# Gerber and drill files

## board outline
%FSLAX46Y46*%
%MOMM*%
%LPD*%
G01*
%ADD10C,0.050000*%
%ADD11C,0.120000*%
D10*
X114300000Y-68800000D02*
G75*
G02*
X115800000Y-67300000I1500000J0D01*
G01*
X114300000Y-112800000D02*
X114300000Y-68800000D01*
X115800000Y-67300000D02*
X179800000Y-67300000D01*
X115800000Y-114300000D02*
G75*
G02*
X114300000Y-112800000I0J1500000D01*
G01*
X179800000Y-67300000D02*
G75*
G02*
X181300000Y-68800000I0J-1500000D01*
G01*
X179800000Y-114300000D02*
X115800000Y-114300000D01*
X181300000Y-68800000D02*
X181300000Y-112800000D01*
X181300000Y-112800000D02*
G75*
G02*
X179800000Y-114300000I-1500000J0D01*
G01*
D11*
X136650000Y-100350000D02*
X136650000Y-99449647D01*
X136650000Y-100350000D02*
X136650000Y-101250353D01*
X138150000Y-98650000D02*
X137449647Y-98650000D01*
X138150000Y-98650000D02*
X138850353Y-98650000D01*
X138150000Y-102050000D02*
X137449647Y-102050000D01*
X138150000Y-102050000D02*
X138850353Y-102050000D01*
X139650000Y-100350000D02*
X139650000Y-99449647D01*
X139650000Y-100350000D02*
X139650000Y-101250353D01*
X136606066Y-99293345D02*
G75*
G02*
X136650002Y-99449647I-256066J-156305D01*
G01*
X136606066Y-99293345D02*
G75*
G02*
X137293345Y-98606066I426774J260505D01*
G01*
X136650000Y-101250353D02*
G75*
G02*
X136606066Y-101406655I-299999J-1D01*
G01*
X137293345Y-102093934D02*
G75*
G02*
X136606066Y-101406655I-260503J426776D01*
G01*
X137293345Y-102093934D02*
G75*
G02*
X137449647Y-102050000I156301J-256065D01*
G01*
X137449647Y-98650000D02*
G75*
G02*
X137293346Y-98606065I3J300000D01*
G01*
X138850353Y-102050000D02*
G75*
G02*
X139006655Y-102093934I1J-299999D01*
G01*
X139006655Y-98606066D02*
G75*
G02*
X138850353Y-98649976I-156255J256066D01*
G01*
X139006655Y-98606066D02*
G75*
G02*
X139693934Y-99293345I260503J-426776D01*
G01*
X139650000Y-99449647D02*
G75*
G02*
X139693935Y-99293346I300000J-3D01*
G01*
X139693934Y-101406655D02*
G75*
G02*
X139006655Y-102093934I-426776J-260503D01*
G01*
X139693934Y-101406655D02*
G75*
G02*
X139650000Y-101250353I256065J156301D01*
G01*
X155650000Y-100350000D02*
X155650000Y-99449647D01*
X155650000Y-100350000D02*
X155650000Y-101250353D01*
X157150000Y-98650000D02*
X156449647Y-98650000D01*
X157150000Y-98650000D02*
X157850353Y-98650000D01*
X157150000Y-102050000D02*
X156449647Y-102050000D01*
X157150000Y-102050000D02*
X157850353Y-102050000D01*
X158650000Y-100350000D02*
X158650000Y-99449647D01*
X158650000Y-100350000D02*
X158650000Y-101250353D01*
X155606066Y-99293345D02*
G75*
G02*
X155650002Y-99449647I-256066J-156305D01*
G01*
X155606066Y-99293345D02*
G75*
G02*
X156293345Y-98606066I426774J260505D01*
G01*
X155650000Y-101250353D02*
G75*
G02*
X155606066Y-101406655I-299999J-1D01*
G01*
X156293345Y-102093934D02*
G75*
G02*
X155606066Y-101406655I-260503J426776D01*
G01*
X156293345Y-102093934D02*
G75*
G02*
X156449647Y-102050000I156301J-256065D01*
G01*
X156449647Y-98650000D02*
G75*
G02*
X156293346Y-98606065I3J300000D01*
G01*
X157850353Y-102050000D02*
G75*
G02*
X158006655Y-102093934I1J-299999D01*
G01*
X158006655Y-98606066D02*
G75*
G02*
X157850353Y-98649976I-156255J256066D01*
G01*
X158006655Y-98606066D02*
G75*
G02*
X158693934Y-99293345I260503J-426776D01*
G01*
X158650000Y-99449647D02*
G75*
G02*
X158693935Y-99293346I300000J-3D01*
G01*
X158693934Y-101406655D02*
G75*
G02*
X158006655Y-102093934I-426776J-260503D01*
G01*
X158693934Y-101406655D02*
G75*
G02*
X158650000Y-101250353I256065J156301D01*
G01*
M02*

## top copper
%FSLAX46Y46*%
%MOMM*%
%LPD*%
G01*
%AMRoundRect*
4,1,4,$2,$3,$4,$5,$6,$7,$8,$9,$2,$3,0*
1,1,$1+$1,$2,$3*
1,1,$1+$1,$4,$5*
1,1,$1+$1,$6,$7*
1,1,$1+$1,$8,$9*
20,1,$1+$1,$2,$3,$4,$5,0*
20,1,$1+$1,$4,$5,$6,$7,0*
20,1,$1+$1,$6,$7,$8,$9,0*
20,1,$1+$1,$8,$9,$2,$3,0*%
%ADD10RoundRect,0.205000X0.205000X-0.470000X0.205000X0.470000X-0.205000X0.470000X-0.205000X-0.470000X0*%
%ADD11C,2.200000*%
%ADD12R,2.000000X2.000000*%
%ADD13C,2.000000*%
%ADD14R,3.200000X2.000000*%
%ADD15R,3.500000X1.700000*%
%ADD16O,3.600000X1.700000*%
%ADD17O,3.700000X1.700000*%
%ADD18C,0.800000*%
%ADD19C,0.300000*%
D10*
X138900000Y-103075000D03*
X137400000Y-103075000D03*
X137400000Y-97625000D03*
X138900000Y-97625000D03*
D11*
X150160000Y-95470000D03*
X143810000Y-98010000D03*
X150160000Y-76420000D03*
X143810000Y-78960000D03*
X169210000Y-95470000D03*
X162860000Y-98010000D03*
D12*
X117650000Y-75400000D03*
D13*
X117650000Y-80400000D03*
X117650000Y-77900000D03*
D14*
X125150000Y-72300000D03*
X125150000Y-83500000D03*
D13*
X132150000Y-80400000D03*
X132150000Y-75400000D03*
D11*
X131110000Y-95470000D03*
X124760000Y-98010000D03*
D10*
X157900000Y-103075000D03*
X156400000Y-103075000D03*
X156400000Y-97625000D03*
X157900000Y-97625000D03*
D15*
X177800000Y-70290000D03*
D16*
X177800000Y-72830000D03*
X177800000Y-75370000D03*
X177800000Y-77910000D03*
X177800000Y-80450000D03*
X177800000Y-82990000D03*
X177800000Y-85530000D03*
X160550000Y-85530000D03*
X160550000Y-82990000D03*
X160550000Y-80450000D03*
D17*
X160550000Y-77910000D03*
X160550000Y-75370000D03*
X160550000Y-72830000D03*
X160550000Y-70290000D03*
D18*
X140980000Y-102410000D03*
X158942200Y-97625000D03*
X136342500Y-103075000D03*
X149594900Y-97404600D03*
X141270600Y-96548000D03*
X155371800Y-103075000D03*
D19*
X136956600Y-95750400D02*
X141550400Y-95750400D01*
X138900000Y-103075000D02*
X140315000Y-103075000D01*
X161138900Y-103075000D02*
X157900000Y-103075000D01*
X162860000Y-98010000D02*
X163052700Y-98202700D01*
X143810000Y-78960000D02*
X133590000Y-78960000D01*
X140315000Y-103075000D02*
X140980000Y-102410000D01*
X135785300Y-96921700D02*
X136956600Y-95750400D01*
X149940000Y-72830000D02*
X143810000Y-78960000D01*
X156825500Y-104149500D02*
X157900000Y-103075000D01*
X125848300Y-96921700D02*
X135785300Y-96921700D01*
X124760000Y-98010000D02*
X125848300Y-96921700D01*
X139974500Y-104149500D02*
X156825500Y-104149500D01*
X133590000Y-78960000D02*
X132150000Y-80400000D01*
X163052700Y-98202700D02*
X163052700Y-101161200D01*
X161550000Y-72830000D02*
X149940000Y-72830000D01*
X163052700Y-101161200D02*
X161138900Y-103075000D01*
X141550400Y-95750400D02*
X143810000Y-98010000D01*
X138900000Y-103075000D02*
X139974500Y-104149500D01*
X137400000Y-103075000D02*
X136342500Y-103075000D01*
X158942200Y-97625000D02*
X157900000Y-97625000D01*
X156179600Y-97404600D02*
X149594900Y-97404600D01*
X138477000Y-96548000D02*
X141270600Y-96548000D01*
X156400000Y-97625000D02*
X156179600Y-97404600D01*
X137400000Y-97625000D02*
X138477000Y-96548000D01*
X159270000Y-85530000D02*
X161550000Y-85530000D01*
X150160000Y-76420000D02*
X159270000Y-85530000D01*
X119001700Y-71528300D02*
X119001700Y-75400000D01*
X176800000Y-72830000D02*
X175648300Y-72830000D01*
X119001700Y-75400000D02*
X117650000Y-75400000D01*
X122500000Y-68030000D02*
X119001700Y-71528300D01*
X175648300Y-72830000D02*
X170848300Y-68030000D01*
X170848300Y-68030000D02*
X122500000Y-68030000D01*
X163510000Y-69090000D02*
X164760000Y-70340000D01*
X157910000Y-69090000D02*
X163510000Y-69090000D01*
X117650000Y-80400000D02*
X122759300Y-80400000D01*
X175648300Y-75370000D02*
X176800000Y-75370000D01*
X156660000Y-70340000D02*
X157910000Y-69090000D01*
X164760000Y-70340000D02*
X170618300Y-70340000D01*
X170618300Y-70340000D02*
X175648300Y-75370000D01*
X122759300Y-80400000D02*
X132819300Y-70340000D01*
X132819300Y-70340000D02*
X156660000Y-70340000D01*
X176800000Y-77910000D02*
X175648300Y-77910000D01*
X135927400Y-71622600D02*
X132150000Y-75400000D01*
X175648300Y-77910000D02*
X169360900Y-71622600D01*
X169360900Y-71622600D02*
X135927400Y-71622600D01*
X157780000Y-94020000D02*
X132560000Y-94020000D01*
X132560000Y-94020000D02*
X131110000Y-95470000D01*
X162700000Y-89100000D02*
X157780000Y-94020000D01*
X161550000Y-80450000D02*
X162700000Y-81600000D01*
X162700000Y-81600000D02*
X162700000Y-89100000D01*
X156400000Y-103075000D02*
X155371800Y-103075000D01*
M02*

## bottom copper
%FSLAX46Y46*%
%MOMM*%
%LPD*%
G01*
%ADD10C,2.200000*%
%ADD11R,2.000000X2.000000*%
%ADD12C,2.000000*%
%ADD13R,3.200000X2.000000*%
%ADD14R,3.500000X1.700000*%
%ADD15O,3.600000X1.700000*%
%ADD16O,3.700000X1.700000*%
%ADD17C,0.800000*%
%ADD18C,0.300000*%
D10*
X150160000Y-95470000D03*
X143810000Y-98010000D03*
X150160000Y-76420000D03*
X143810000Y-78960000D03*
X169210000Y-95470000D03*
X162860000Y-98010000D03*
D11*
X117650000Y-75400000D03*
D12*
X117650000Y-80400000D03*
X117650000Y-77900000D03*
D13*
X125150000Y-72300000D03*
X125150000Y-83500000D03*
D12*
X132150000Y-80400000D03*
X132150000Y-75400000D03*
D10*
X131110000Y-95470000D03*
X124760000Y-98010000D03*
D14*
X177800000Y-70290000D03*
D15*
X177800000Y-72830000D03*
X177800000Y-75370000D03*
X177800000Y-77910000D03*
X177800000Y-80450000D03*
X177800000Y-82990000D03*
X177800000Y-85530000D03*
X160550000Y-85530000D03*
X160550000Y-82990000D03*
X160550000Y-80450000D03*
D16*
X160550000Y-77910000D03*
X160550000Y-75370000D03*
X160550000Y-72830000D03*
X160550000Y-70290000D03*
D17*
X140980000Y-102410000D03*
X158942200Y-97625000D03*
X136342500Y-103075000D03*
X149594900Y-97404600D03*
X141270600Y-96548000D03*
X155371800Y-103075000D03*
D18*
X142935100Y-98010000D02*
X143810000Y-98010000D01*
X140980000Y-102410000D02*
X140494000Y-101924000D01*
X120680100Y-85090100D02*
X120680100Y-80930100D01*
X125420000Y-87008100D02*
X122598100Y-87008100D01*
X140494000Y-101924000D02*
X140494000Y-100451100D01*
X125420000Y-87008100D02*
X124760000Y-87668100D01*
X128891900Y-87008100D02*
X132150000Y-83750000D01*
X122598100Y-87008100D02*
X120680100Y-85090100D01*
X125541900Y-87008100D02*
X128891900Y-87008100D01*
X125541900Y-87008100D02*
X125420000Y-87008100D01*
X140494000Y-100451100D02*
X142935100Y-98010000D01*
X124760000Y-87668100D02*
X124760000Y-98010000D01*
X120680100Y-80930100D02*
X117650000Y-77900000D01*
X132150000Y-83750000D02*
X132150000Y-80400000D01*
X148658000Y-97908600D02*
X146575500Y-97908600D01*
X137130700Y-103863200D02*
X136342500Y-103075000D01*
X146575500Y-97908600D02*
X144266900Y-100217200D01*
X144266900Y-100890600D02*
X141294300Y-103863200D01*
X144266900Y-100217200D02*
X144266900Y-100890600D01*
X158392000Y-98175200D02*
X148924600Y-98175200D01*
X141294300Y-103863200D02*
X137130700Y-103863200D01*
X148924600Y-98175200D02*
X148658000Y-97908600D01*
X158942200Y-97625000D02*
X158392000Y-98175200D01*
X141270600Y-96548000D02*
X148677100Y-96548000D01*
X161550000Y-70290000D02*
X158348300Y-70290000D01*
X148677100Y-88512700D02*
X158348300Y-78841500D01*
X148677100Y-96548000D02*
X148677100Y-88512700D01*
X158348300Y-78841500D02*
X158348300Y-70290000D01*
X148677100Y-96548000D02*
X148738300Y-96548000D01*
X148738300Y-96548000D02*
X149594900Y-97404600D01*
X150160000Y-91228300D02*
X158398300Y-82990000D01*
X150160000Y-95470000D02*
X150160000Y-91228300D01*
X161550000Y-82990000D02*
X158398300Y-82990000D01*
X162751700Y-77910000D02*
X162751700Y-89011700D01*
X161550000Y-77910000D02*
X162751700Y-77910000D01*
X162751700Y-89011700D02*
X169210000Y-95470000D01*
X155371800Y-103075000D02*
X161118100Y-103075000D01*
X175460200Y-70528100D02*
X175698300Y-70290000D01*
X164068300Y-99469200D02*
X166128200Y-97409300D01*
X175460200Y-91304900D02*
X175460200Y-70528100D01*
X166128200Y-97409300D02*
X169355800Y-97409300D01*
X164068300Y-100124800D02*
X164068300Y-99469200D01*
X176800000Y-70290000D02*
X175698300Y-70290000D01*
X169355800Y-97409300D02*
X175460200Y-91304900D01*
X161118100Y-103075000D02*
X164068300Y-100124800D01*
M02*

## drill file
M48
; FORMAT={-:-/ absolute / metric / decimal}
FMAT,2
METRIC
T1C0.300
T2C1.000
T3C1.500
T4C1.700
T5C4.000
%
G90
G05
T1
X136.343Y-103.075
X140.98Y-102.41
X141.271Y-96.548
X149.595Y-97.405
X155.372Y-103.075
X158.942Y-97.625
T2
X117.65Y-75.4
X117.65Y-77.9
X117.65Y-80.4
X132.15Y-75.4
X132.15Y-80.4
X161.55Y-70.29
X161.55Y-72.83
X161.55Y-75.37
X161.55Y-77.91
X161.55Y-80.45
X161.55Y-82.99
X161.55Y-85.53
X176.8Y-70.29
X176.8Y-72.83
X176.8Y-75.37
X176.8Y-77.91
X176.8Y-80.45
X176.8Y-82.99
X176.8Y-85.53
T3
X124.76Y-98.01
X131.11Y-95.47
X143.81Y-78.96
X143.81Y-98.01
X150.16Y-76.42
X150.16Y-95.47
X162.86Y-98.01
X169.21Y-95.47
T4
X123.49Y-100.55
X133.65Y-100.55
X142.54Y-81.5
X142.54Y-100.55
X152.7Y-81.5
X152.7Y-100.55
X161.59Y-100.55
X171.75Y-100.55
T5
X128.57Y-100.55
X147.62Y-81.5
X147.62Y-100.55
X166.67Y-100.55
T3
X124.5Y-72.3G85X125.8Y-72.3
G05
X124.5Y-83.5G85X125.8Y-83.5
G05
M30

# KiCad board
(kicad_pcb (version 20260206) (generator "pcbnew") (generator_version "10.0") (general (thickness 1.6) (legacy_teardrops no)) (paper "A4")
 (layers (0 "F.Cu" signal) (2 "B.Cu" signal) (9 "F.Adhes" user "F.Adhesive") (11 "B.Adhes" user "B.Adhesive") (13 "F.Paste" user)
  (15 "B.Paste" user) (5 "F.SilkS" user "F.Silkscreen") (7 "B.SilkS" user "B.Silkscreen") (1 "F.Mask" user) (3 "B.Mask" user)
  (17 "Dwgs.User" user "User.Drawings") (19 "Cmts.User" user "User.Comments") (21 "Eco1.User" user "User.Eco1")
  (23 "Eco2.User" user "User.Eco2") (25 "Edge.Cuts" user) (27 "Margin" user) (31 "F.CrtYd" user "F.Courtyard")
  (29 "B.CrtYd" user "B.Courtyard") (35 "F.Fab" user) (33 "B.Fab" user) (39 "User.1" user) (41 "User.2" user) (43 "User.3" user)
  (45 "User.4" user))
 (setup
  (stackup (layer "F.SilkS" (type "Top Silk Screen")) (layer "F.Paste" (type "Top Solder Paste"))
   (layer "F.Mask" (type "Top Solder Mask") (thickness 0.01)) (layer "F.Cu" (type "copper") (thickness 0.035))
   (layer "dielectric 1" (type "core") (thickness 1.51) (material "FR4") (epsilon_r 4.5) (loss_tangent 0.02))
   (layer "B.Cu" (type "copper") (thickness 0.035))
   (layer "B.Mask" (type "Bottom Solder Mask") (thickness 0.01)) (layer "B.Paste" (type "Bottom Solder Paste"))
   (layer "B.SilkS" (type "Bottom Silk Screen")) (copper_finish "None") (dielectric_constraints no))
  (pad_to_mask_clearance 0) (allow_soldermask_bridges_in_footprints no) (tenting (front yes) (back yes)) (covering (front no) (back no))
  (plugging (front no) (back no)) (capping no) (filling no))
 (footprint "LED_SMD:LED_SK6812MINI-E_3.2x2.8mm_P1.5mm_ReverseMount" (layer "F.Cu") (at 138.15 100.35 90)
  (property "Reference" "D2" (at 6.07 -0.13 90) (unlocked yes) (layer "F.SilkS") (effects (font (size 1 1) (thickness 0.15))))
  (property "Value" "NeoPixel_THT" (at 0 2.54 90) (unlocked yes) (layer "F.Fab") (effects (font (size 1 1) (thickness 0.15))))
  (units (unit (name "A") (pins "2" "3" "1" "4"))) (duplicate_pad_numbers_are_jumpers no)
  (fp_line (start 0 -1.5) (end 0.900353 -1.5) (stroke (width 0.12) (type solid)) (layer "Edge.Cuts"))
  (fp_line (start 0 -1.5) (end -0.900353 -1.5) (stroke (width 0.12) (type solid)) (layer "Edge.Cuts"))
  (fp_line (start 1.7 0) (end 1.7 -0.700353) (stroke (width 0.12) (type solid)) (layer "Edge.Cuts"))
  (fp_line (start 1.7 0) (end 1.7 0.700353) (stroke (width 0.12) (type solid)) (layer "Edge.Cuts"))
  (fp_line (start -1.7 0) (end -1.7 -0.700353) (stroke (width 0.12) (type solid)) (layer "Edge.Cuts"))
  (fp_line (start -1.7 0) (end -1.7 0.700353) (stroke (width 0.12) (type solid)) (layer "Edge.Cuts"))
  (fp_line (start 0 1.5) (end 0.900353 1.5) (stroke (width 0.12) (type solid)) (layer "Edge.Cuts"))
  (fp_line (start 0 1.5) (end -0.900353 1.5) (stroke (width 0.12) (type solid)) (layer "Edge.Cuts"))
  (fp_arc (start 1.056655 -1.543934) (mid 0.981532 -1.511192) (end 0.900353 -1.5) (stroke (width 0.12) (type solid)) (layer "Edge.Cuts"))
  (fp_arc (start 1.056655 -1.543934) (mid 1.670711 -1.470711) (end 1.743934 -0.856655) (stroke (width 0.12) (type solid))
   (layer "Edge.Cuts"))
  (fp_arc (start -0.900353 -1.5) (mid -0.981532 -1.511192) (end -1.056655 -1.543934) (stroke (width 0.12) (type solid)) (layer "Edge.Cuts"))
  (fp_arc (start -1.743934 -0.856655) (mid -1.670711 -1.470711) (end -1.056655 -1.543934) (stroke (width 0.12) (type solid))
   (layer "Edge.Cuts"))
  (fp_arc (start -1.743934 -0.856655) (mid -1.711192 -0.781532) (end -1.7 -0.700353) (stroke (width 0.12) (type solid)) (layer "Edge.Cuts"))
  (fp_arc (start 1.7 -0.700353) (mid 1.711192 -0.781532) (end 1.743934 -0.856655) (stroke (width 0.12) (type solid)) (layer "Edge.Cuts"))
  (fp_arc (start -1.7 0.700353) (mid -1.711192 0.781532) (end -1.743934 0.856655) (stroke (width 0.12) (type solid)) (layer "Edge.Cuts"))
  (fp_arc (start 1.743934 0.856655) (mid 1.711192 0.781532) (end 1.7 0.700353) (stroke (width 0.12) (type solid)) (layer "Edge.Cuts"))
  (fp_arc (start 1.743934 0.856655) (mid 1.670711 1.470711) (end 1.056655 1.543934) (stroke (width 0.12) (type solid)) (layer "Edge.Cuts"))
  (fp_arc (start 0.900353 1.5) (mid 0.981532 1.511192) (end 1.056655 1.543934) (stroke (width 0.12) (type solid)) (layer "Edge.Cuts"))
  (fp_arc (start -1.056655 1.543934) (mid -1.670711 1.470711) (end -1.743934 0.856655) (stroke (width 0.12) (type solid))
   (layer "Edge.Cuts"))
  (fp_arc (start -1.056655 1.543934) (mid -0.981532 1.511192) (end -0.900353 1.5) (stroke (width 0.12) (type solid)) (layer "Edge.Cuts"))
  (pad "1" smd roundrect (at -2.725 0.75 90) (size 1.35 0.82) (layers "F.Cu" "F.Mask" "F.Paste") (roundrect_rratio 0.25) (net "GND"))
  (pad "2" smd roundrect (at -2.725 -0.75 90) (size 1.35 0.82) (layers "F.Cu" "F.Mask" "F.Paste") (roundrect_rratio 0.25)
   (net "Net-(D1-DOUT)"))
  (pad "3" smd roundrect (at 2.725 -0.75 90) (size 1.35 0.82) (layers "F.Cu" "F.Mask" "F.Paste") (roundrect_rratio 0.25) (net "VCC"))
  (pad "4" smd roundrect (at 2.725 0.75 90) (size 1.35 0.82) (layers "F.Cu" "F.Mask" "F.Paste") (roundrect_rratio 0.25)
   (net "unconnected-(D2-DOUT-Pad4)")))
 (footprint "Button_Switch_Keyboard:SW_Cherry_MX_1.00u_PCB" (layer "F.Cu") (at 150.16 95.47)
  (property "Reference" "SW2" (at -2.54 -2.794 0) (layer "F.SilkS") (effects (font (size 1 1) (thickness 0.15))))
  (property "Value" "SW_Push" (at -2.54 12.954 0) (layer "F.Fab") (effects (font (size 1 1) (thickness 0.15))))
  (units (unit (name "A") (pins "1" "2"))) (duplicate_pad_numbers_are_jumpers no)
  (pad "" np_thru_hole circle (at -7.62 5.08) (size 1.7 1.7) (drill 1.7) (layers "*.Cu" "*.Mask"))
  (pad "" np_thru_hole circle (at -2.54 5.08) (size 4 4) (drill 4) (layers "*.Cu" "*.Mask"))
  (pad "" np_thru_hole circle (at 2.54 5.08) (size 1.7 1.7) (drill 1.7) (layers "*.Cu" "*.Mask"))
  (pad "1" thru_hole circle (at 0 0) (size 2.2 2.2) (drill 1.5) (layers "*.Cu" "*.Mask") (remove_unused_layers no)
   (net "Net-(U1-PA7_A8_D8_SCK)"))
  (pad "2" thru_hole circle (at -6.35 2.54) (size 2.2 2.2) (drill 1.5) (layers "*.Cu" "*.Mask") (remove_unused_layers no) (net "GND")))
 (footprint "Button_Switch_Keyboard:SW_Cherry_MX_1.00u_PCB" (layer "F.Cu") (at 150.16 76.42)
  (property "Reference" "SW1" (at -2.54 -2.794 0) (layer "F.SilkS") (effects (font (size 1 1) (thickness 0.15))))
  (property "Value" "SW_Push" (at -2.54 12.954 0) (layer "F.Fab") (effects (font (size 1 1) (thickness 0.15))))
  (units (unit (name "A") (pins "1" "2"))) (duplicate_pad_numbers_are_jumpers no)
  (pad "" np_thru_hole circle (at -7.62 5.08) (size 1.7 1.7) (drill 1.7) (layers "*.Cu" "*.Mask"))
  (pad "" np_thru_hole circle (at -2.54 5.08) (size 4 4) (drill 4) (layers "*.Cu" "*.Mask"))
  (pad "" np_thru_hole circle (at 2.54 5.08) (size 1.7 1.7) (drill 1.7) (layers "*.Cu" "*.Mask"))
  (pad "1" thru_hole circle (at 0 0) (size 2.2 2.2) (drill 1.5) (layers "*.Cu" "*.Mask") (remove_unused_layers no)
   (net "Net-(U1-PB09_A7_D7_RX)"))
  (pad "2" thru_hole circle (at -6.35 2.54) (size 2.2 2.2) (drill 1.5) (layers "*.Cu" "*.Mask") (remove_unused_layers no) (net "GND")))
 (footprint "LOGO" (layer "F.Cu") (at 176.41 109.06)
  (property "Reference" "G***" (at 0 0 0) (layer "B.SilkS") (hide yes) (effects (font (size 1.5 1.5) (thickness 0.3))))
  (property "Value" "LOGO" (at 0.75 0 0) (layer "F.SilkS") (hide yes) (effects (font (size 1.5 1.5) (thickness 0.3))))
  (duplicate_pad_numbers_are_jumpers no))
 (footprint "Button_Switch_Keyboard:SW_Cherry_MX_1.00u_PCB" (layer "F.Cu") (at 169.21 95.47)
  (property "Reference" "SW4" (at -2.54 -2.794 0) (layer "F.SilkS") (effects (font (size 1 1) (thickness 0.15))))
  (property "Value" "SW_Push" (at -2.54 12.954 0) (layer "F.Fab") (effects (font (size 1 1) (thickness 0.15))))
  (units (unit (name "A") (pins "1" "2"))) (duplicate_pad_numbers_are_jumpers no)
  (pad "" np_thru_hole circle (at -7.62 5.08) (size 1.7 1.7) (drill 1.7) (layers "*.Cu" "*.Mask"))
  (pad "" np_thru_hole circle (at -2.54 5.08) (size 4 4) (drill 4) (layers "*.Cu" "*.Mask"))
  (pad "" np_thru_hole circle (at 2.54 5.08) (size 1.7 1.7) (drill 1.7) (layers "*.Cu" "*.Mask"))
  (pad "1" thru_hole circle (at 0 0) (size 2.2 2.2) (drill 1.5) (layers "*.Cu" "*.Mask") (remove_unused_layers no)
   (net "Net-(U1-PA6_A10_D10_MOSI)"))
  (pad "2" thru_hole circle (at -6.35 2.54) (size 2.2 2.2) (drill 1.5) (layers "*.Cu" "*.Mask") (remove_unused_layers no) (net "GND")))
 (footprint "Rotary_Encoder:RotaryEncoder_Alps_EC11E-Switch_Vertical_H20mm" (layer "F.Cu") (at 117.65 75.4)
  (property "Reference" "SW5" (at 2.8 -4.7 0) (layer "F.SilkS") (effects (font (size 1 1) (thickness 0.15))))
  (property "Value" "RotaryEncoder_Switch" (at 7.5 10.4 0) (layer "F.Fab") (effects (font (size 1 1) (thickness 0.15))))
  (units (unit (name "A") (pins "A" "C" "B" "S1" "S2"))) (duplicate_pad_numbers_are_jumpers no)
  (pad "A" thru_hole rect (at 0 0) (size 2 2) (drill 1) (layers "*.Cu" "*.Mask") (remove_unused_layers no) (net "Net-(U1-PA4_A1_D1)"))
  (pad "B" thru_hole circle (at 0 5) (size 2 2) (drill 1) (layers "*.Cu" "*.Mask") (remove_unused_layers no) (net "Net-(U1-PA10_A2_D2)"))
  (pad "C" thru_hole circle (at 0 2.5) (size 2 2) (drill 1) (layers "*.Cu" "*.Mask") (remove_unused_layers no) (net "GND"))
  (pad "MP" thru_hole rect (at 7.5 -3.1) (size 3.2 2) (drill oval 2.8 1.5) (layers "*.Cu" "*.Mask") (remove_unused_layers no))
  (pad "MP" thru_hole rect (at 7.5 8.1) (size 3.2 2) (drill oval 2.8 1.5) (layers "*.Cu" "*.Mask") (remove_unused_layers no))
  (pad "S1" thru_hole circle (at 14.5 5) (size 2 2) (drill 1) (layers "*.Cu" "*.Mask") (remove_unused_layers no) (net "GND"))
  (pad "S2" thru_hole circle (at 14.5 0) (size 2 2) (drill 1) (layers "*.Cu" "*.Mask") (remove_unused_layers no) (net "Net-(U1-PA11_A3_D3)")))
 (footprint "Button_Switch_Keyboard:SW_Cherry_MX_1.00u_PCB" (layer "F.Cu") (at 131.11 95.47)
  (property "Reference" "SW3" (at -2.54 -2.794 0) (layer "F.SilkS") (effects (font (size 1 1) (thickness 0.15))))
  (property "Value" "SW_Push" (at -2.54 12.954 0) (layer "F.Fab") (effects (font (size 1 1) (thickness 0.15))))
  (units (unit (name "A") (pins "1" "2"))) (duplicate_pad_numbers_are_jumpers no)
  (pad "" np_thru_hole circle (at -7.62 5.08) (size 1.7 1.7) (drill 1.7) (layers "*.Cu" "*.Mask"))
  (pad "" np_thru_hole circle (at -2.54 5.08) (size 4 4) (drill 4) (layers "*.Cu" "*.Mask"))
  (pad "" np_thru_hole circle (at 2.54 5.08) (size 1.7 1.7) (drill 1.7) (layers "*.Cu" "*.Mask"))
  (pad "1" thru_hole circle (at 0 0) (size 2.2 2.2) (drill 1.5) (layers "*.Cu" "*.Mask") (remove_unused_layers no)
   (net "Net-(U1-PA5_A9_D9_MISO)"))
  (pad "2" thru_hole circle (at -6.35 2.54) (size 2.2 2.2) (drill 1.5) (layers "*.Cu" "*.Mask") (remove_unused_layers no) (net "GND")))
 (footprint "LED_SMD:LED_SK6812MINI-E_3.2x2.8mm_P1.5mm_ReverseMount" (layer "F.Cu") (at 157.15 100.35 90)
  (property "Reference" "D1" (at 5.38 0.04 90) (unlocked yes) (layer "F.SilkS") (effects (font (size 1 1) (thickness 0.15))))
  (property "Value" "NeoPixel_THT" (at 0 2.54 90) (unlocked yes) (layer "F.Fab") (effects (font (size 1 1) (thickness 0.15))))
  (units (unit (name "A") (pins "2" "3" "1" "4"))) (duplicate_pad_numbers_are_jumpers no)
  (fp_line (start 0 -1.5) (end 0.900353 -1.5) (stroke (width 0.12) (type solid)) (layer "Edge.Cuts"))
  (fp_line (start 0 -1.5) (end -0.900353 -1.5) (stroke (width 0.12) (type solid)) (layer "Edge.Cuts"))
  (fp_line (start 1.7 0) (end 1.7 -0.700353) (stroke (width 0.12) (type solid)) (layer "Edge.Cuts"))
  (fp_line (start 1.7 0) (end 1.7 0.700353) (stroke (width 0.12) (type solid)) (layer "Edge.Cuts"))
  (fp_line (start -1.7 0) (end -1.7 -0.700353) (stroke (width 0.12) (type solid)) (layer "Edge.Cuts"))
  (fp_line (start -1.7 0) (end -1.7 0.700353) (stroke (width 0.12) (type solid)) (layer "Edge.Cuts"))
  (fp_line (start 0 1.5) (end 0.900353 1.5) (stroke (width 0.12) (type solid)) (layer "Edge.Cuts"))
  (fp_line (start 0 1.5) (end -0.900353 1.5) (stroke (width 0.12) (type solid)) (layer "Edge.Cuts"))
  (fp_arc (start 1.056655 -1.543934) (mid 0.981532 -1.511192) (end 0.900353 -1.5) (stroke (width 0.12) (type solid)) (layer "Edge.Cuts"))
  (fp_arc (start 1.056655 -1.543934) (mid 1.670711 -1.470711) (end 1.743934 -0.856655) (stroke (width 0.12) (type solid))
   (layer "Edge.Cuts"))
  (fp_arc (start -0.900353 -1.5) (mid -0.981532 -1.511192) (end -1.056655 -1.543934) (stroke (width 0.12) (type solid)) (layer "Edge.Cuts"))
  (fp_arc (start -1.743934 -0.856655) (mid -1.670711 -1.470711) (end -1.056655 -1.543934) (stroke (width 0.12) (type solid))
   (layer "Edge.Cuts"))
  (fp_arc (start -1.743934 -0.856655) (mid -1.711192 -0.781532) (end -1.7 -0.700353) (stroke (width 0.12) (type solid)) (layer "Edge.Cuts"))
  (fp_arc (start 1.7 -0.700353) (mid 1.711192 -0.781532) (end 1.743934 -0.856655) (stroke (width 0.12) (type solid)) (layer "Edge.Cuts"))
  (fp_arc (start -1.7 0.700353) (mid -1.711192 0.781532) (end -1.743934 0.856655) (stroke (width 0.12) (type solid)) (layer "Edge.Cuts"))
  (fp_arc (start 1.743934 0.856655) (mid 1.711192 0.781532) (end 1.7 0.700353) (stroke (width 0.12) (type solid)) (layer "Edge.Cuts"))
  (fp_arc (start 1.743934 0.856655) (mid 1.670711 1.470711) (end 1.056655 1.543934) (stroke (width 0.12) (type solid)) (layer "Edge.Cuts"))
  (fp_arc (start 0.900353 1.5) (mid 0.981532 1.511192) (end 1.056655 1.543934) (stroke (width 0.12) (type solid)) (layer "Edge.Cuts"))
  (fp_arc (start -1.056655 1.543934) (mid -1.670711 1.470711) (end -1.743934 0.856655) (stroke (width 0.12) (type solid))
   (layer "Edge.Cuts"))
  (fp_arc (start -1.056655 1.543934) (mid -0.981532 1.511192) (end -0.900353 1.5) (stroke (width 0.12) (type solid)) (layer "Edge.Cuts"))
  (pad "1" smd roundrect (at -2.725 0.75 90) (size 1.35 0.82) (layers "F.Cu" "F.Mask" "F.Paste") (roundrect_rratio 0.25) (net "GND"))
  (pad "2" smd roundrect (at -2.725 -0.75 90) (size 1.35 0.82) (layers "F.Cu" "F.Mask" "F.Paste") (roundrect_rratio 0.25)
   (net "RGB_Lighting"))
  (pad "3" smd roundrect (at 2.725 -0.75 90) (size 1.35 0.82) (layers "F.Cu" "F.Mask" "F.Paste") (roundrect_rratio 0.25) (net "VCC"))
  (pad "4" smd roundrect (at 2.725 0.75 90) (size 1.35 0.82) (layers "F.Cu" "F.Mask" "F.Paste") (roundrect_rratio 0.25)
   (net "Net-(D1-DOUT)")))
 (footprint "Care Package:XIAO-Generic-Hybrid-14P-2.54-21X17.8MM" (layer "B.Cu") (at 169.175 77.91 180)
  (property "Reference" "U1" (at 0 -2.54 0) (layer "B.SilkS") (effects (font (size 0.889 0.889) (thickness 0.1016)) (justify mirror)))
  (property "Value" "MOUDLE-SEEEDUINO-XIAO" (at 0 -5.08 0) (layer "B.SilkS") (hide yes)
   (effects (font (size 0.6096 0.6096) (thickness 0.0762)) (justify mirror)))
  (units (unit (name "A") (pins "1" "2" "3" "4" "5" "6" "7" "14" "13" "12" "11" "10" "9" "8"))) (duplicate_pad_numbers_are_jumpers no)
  (pad "1" thru_hole rect (at -7.625 7.62 180) (size 3.5 1.7) (drill 1 (offset -1 0)) (layers "*.Cu" "*.Mask") (remove_unused_layers no)
   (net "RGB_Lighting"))
  (pad "2" thru_hole oval (at -7.625 5.08 180) (size 3.6 1.7) (drill 1 (offset -1 0)) (layers "*.Cu" "*.Mask") (remove_unused_layers no)
   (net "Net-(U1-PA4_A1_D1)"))
  (pad "3" thru_hole oval (at -7.625 2.54 180) (size 3.6 1.7) (drill 1 (offset -1 0)) (layers "*.Cu" "*.Mask") (remove_unused_layers no)
   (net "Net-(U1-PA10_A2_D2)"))
  (pad "4" thru_hole oval (at -7.625 0 180) (size 3.6 1.7) (drill 1 (offset -1 0)) (layers "*.Cu" "*.Mask") (remove_unused_layers no)
   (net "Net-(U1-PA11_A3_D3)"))
  (pad "5" thru_hole oval (at -7.625 -2.54 180) (size 3.6 1.7) (drill 1 (offset -1 0)) (layers "*.Cu" "*.Mask") (remove_unused_layers no)
   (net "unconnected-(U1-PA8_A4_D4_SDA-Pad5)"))
  (pad "6" thru_hole oval (at -7.625 -5.08) (size 3.6 1.7) (drill 1 (offset 1 0)) (layers "*.Cu" "*.Mask") (remove_unused_layers no)
   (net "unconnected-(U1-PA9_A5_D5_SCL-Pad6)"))
  (pad "7" thru_hole oval (at -7.625 -7.62 180) (size 3.6 1.7) (drill 1 (offset -1 0)) (layers "*.Cu" "*.Mask") (remove_unused_layers no)
   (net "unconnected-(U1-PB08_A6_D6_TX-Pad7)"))
  (pad "8" thru_hole oval (at 7.625 -7.62 180) (size 3.6 1.7) (drill 1 (offset 1 0)) (layers "*.Cu" "*.Mask") (remove_unused_layers no)
   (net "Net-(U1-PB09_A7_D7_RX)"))
  (pad "9" thru_hole oval (at 7.625 -5.08 180) (size 3.6 1.7) (drill 1 (offset 1 0)) (layers "*.Cu" "*.Mask") (remove_unused_layers no)
   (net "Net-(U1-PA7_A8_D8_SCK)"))
  (pad "10" thru_hole oval (at 7.625 -2.54 180) (size 3.6 1.7) (drill 1 (offset 1 0)) (layers "*.Cu" "*.Mask") (remove_unused_layers no)
   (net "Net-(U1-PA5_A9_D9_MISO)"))
  (pad "11" thru_hole oval (at 7.625 0 180) (size 3.7 1.7) (drill 1 (offset 1 0)) (layers "*.Cu" "*.Mask") (remove_unused_layers no)
   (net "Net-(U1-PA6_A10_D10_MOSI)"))
  (pad "12" thru_hole oval (at 7.625 2.54 180) (size 3.7 1.7) (drill 1 (offset 1 0)) (layers "*.Cu" "*.Mask") (remove_unused_layers no)
   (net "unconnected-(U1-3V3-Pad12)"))
  (pad "13" thru_hole oval (at 7.625 5.08 180) (size 3.7 1.7) (drill 1 (offset 1 0)) (layers "*.Cu" "*.Mask") (remove_unused_layers no)
   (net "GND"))
  (pad "14" thru_hole oval (at 7.625 7.62 180) (size 3.7 1.7) (drill 1 (offset 1 0)) (layers "*.Cu" "*.Mask") (remove_unused_layers no)
   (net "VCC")))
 (gr_arc (start 114.3 68.8) (mid 114.73934 67.73934) (end 115.8 67.3) (stroke (width 0.05) (type default)) (layer "Edge.Cuts"))
 (gr_line (start 114.3 112.8) (end 114.3 68.8) (stroke (width 0.05) (type default)) (layer "Edge.Cuts"))
 (gr_line (start 115.8 67.3) (end 179.8 67.3) (stroke (width 0.05) (type default)) (layer "Edge.Cuts"))
 (gr_arc (start 115.8 114.3) (mid 114.73934 113.86066) (end 114.3 112.8) (stroke (width 0.05) (type default)) (layer "Edge.Cuts"))
 (gr_arc (start 179.8 67.3) (mid 180.86066 67.73934) (end 181.3 68.8) (stroke (width 0.05) (type default)) (layer "Edge.Cuts"))
 (gr_line (start 179.8 114.3) (end 115.8 114.3) (stroke (width 0.05) (type default)) (layer "Edge.Cuts"))
 (gr_line (start 181.3 68.8) (end 181.3 112.8) (stroke (width 0.05) (type default)) (layer "Edge.Cuts"))
 (gr_arc (start 181.3 112.8) (mid 180.86066 113.86066) (end 179.8 114.3) (stroke (width 0.05) (type default)) (layer "Edge.Cuts"))
 (segment (start 136.9566 95.7504) (end 141.5504 95.7504) (width 0.3) (layer "F.Cu") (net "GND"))
 (segment (start 138.9 103.075) (end 140.315 103.075) (width 0.3) (layer "F.Cu") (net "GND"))
 (segment (start 161.1389 103.075) (end 157.9 103.075) (width 0.3) (layer "F.Cu") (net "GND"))
 (segment (start 162.86 98.01) (end 163.0527 98.2027) (width 0.3) (layer "F.Cu") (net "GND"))
 (segment (start 143.81 78.96) (end 133.59 78.96) (width 0.3) (layer "F.Cu") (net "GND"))
 (segment (start 140.315 103.075) (end 140.98 102.41) (width 0.3) (layer "F.Cu") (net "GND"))
 (segment (start 135.7853 96.9217) (end 136.9566 95.7504) (width 0.3) (layer "F.Cu") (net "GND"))
 (segment (start 149.94 72.83) (end 143.81 78.96) (width 0.3) (layer "F.Cu") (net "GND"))
 (segment (start 156.8255 104.1495) (end 157.9 103.075) (width 0.3) (layer "F.Cu") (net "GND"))
 (segment (start 125.8483 96.9217) (end 135.7853 96.9217) (width 0.3) (layer "F.Cu") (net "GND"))
 (segment (start 124.76 98.01) (end 125.8483 96.9217) (width 0.3) (layer "F.Cu") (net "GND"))
 (segment (start 139.9745 104.1495) (end 156.8255 104.1495) (width 0.3) (layer "F.Cu") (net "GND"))
 (segment (start 133.59 78.96) (end 132.15 80.4) (width 0.3) (layer "F.Cu") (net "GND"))
 (segment (start 163.0527 98.2027) (end 163.0527 101.1612) (width 0.3) (layer "F.Cu") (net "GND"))
 (segment (start 161.55 72.83) (end 149.94 72.83) (width 0.3) (layer "F.Cu") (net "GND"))
 (segment (start 163.0527 101.1612) (end 161.1389 103.075) (width 0.3) (layer "F.Cu") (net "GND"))
 (segment (start 141.5504 95.7504) (end 143.81 98.01) (width 0.3) (layer "F.Cu") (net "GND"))
 (segment (start 138.9 103.075) (end 139.9745 104.1495) (width 0.3) (layer "F.Cu") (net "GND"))
 (via (at 140.98 102.41) (size 0.8) (drill 0.3) (layers "F.Cu" "B.Cu") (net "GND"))
 (segment (start 142.9351 98.01) (end 143.81 98.01) (width 0.3) (layer "B.Cu") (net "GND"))
 (segment (start 140.98 102.41) (end 140.494 101.924) (width 0.3) (layer "B.Cu") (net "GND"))
 (segment (start 120.6801 85.0901) (end 120.6801 80.9301) (width 0.3) (layer "B.Cu") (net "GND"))
 (segment (start 125.42 87.0081) (end 122.5981 87.0081) (width 0.3) (layer "B.Cu") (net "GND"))
 (segment (start 140.494 101.924) (end 140.494 100.4511) (width 0.3) (layer "B.Cu") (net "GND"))
 (segment (start 125.42 87.0081) (end 124.76 87.6681) (width 0.3) (layer "B.Cu") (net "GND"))
 (segment (start 128.8919 87.0081) (end 132.15 83.75) (width 0.3) (layer "B.Cu") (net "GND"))
 (segment (start 122.5981 87.0081) (end 120.6801 85.0901) (width 0.3) (layer "B.Cu") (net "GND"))
 (segment (start 125.5419 87.0081) (end 128.8919 87.0081) (width 0.3) (layer "B.Cu") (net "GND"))
 (segment (start 125.5419 87.0081) (end 125.42 87.0081) (width 0.3) (layer "B.Cu") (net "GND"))
 (segment (start 140.494 100.4511) (end 142.9351 98.01) (width 0.3) (layer "B.Cu") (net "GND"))
 (segment (start 124.76 87.6681) (end 124.76 98.01) (width 0.3) (layer "B.Cu") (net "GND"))
 (segment (start 120.6801 80.9301) (end 117.65 77.9) (width 0.3) (layer "B.Cu") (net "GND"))
 (segment (start 132.15 83.75) (end 132.15 80.4) (width 0.3) (layer "B.Cu") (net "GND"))
 (segment (start 137.4 103.075) (end 136.3425 103.075) (width 0.3) (layer "F.Cu") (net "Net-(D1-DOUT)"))
 (segment (start 158.9422 97.625) (end 157.9 97.625) (width 0.3) (layer "F.Cu") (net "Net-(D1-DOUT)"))
 (via (at 158.9422 97.625) (size 0.8) (drill 0.3) (layers "F.Cu" "B.Cu") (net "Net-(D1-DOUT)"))
 (via (at 136.3425 103.075) (size 0.8) (drill 0.3) (layers "F.Cu" "B.Cu") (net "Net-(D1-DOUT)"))
 (segment (start 148.658 97.9086) (end 146.5755 97.9086) (width 0.3) (layer "B.Cu") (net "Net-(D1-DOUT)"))
 (segment (start 137.1307 103.8632) (end 136.3425 103.075) (width 0.3) (layer "B.Cu") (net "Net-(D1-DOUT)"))
 (segment (start 146.5755 97.9086) (end 144.2669 100.2172) (width 0.3) (layer "B.Cu") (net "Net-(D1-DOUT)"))
 (segment (start 144.2669 100.8906) (end 141.2943 103.8632) (width 0.3) (layer "B.Cu") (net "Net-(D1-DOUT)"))
 (segment (start 144.2669 100.2172) (end 144.2669 100.8906) (width 0.3) (layer "B.Cu") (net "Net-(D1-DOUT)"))
 (segment (start 158.392 98.1752) (end 148.9246 98.1752) (width 0.3) (layer "B.Cu") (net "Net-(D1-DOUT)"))
 (segment (start 141.2943 103.8632) (end 137.1307 103.8632) (width 0.3) (layer "B.Cu") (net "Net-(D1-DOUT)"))
 (segment (start 148.9246 98.1752) (end 148.658 97.9086) (width 0.3) (layer "B.Cu") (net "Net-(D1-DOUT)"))
 (segment (start 158.9422 97.625) (end 158.392 98.1752) (width 0.3) (layer "B.Cu") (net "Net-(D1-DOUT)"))
 (segment (start 156.1796 97.4046) (end 149.5949 97.4046) (width 0.3) (layer "F.Cu") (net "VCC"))
 (segment (start 138.477 96.548) (end 141.2706 96.548) (width 0.3) (layer "F.Cu") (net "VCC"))
 (segment (start 156.4 97.625) (end 156.1796 97.4046) (width 0.3) (layer "F.Cu") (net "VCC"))
 (segment (start 137.4 97.625) (end 138.477 96.548) (width 0.3) (layer "F.Cu") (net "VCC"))
 (via (at 149.5949 97.4046) (size 0.8) (drill 0.3) (layers "F.Cu" "B.Cu") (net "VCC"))
 (via (at 141.2706 96.548) (size 0.8) (drill 0.3) (layers "F.Cu" "B.Cu") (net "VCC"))
 (segment (start 141.2706 96.548) (end 148.6771 96.548) (width 0.3) (layer "B.Cu") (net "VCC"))
 (segment (start 161.55 70.29) (end 158.3483 70.29) (width 0.3) (layer "B.Cu") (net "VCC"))
 (segment (start 148.6771 88.5127) (end 158.3483 78.8415) (width 0.3) (layer "B.Cu") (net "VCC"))
 (segment (start 148.6771 96.548) (end 148.6771 88.5127) (width 0.3) (layer "B.Cu") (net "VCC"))
 (segment (start 158.3483 78.8415) (end 158.3483 70.29) (width 0.3) (layer "B.Cu") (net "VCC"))
 (segment (start 148.6771 96.548) (end 148.7383 96.548) (width 0.3) (layer "B.Cu") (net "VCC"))
 (segment (start 148.7383 96.548) (end 149.5949 97.4046) (width 0.3) (layer "B.Cu") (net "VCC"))
 (segment (start 150.16 91.2283) (end 158.3983 82.99) (width 0.3) (layer "B.Cu") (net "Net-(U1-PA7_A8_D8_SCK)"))
 (segment (start 150.16 95.47) (end 150.16 91.2283) (width 0.3) (layer "B.Cu") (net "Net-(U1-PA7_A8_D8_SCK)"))
 (segment (start 161.55 82.99) (end 158.3983 82.99) (width 0.3) (layer "B.Cu") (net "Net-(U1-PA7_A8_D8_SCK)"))
 (segment (start 159.27 85.53) (end 161.55 85.53) (width 0.3) (layer "F.Cu") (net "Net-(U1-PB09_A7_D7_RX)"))
 (segment (start 150.16 76.42) (end 159.27 85.53) (width 0.3) (layer "F.Cu") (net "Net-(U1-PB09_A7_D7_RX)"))
 (segment (start 162.7517 77.91) (end 162.7517 89.0117) (width 0.3) (layer "B.Cu") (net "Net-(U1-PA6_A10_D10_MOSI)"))
 (segment (start 161.55 77.91) (end 162.7517 77.91) (width 0.3) (layer "B.Cu") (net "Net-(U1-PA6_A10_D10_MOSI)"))
 (segment (start 162.7517 89.0117) (end 169.21 95.47) (width 0.3) (layer "B.Cu") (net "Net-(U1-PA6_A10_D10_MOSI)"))
 (segment (start 119.0017 71.5283) (end 119.0017 75.4) (width 0.3) (layer "F.Cu") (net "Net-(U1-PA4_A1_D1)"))
 (segment (start 176.8 72.83) (end 175.6483 72.83) (width 0.3) (layer "F.Cu") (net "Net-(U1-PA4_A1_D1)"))
 (segment (start 119.0017 75.4) (end 117.65 75.4) (width 0.3) (layer "F.Cu") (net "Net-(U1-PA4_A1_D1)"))
 (segment (start 122.5 68.03) (end 119.0017 71.5283) (width 0.3) (layer "F.Cu") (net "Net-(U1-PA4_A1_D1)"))
 (segment (start 175.6483 72.83) (end 170.8483 68.03) (width 0.3) (layer "F.Cu") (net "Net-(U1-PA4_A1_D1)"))
 (segment (start 170.8483 68.03) (end 122.5 68.03) (width 0.3) (layer "F.Cu") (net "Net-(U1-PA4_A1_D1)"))
 (segment (start 163.51 69.09) (end 164.76 70.34) (width 0.3) (layer "F.Cu") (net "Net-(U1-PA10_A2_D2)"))
 (segment (start 157.91 69.09) (end 163.51 69.09) (width 0.3) (layer "F.Cu") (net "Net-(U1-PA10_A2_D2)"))
 (segment (start 117.65 80.4) (end 122.7593 80.4) (width 0.3) (layer "F.Cu") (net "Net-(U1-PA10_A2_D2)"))
 (segment (start 175.6483 75.37) (end 176.8 75.37) (width 0.3) (layer "F.Cu") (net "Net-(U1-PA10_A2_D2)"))
 (segment (start 156.66 70.34) (end 157.91 69.09) (width 0.3) (layer "F.Cu") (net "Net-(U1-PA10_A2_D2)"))
 (segment (start 164.76 70.34) (end 170.6183 70.34) (width 0.3) (layer "F.Cu") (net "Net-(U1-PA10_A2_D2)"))
 (segment (start 170.6183 70.34) (end 175.6483 75.37) (width 0.3) (layer "F.Cu") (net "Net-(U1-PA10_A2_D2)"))
 (segment (start 122.7593 80.4) (end 132.8193 70.34) (width 0.3) (layer "F.Cu") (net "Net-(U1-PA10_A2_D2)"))
 (segment (start 132.8193 70.34) (end 156.66 70.34) (width 0.3) (layer "F.Cu") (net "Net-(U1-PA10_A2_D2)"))
 (segment (start 176.8 77.91) (end 175.6483 77.91) (width 0.3) (layer "F.Cu") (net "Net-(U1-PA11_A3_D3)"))
 (segment (start 135.9274 71.6226) (end 132.15 75.4) (width 0.3) (layer "F.Cu") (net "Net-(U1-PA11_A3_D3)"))
 (segment (start 175.6483 77.91) (end 169.3609 71.6226) (width 0.3) (layer "F.Cu") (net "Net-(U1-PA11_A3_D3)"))
 (segment (start 169.3609 71.6226) (end 135.9274 71.6226) (width 0.3) (layer "F.Cu") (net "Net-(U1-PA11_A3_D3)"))
 (segment (start 157.78 94.02) (end 132.56 94.02) (width 0.3) (layer "F.Cu") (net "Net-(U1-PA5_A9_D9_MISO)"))
 (segment (start 132.56 94.02) (end 131.11 95.47) (width 0.3) (layer "F.Cu") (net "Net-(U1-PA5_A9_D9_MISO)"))
 (segment (start 162.7 89.1) (end 157.78 94.02) (width 0.3) (layer "F.Cu") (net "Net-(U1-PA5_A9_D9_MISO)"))
 (segment (start 161.55 80.45) (end 162.7 81.6) (width 0.3) (layer "F.Cu") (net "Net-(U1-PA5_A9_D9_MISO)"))
 (segment (start 162.7 81.6) (end 162.7 89.1) (width 0.3) (layer "F.Cu") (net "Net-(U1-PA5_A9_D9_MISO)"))
 (segment (start 156.4 103.075) (end 155.3718 103.075) (width 0.3) (layer "F.Cu") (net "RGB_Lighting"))
 (via (at 155.3718 103.075) (size 0.8) (drill 0.3) (layers "F.Cu" "B.Cu") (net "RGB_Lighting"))
 (segment (start 155.3718 103.075) (end 161.1181 103.075) (width 0.3) (layer "B.Cu") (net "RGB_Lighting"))
 (segment (start 175.4602 70.5281) (end 175.6983 70.29) (width 0.3) (layer "B.Cu") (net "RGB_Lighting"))
 (segment (start 164.0683 99.4692) (end 166.1282 97.4093) (width 0.3) (layer "B.Cu") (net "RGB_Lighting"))
 (segment (start 175.4602 91.3049) (end 175.4602 70.5281) (width 0.3) (layer "B.Cu") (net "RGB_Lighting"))
 (segment (start 166.1282 97.4093) (end 169.3558 97.4093) (width 0.3) (layer "B.Cu") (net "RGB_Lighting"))
 (segment (start 164.0683 100.1248) (end 164.0683 99.4692) (width 0.3) (layer "B.Cu") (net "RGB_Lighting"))
 (segment (start 176.8 70.29) (end 175.6983 70.29) (width 0.3) (layer "B.Cu") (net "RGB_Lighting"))
 (segment (start 169.3558 97.4093) (end 175.4602 91.3049) (width 0.3) (layer "B.Cu") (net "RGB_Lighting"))
 (segment (start 161.1181 103.075) (end 164.0683 100.1248) (width 0.3) (layer "B.Cu") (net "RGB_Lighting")))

